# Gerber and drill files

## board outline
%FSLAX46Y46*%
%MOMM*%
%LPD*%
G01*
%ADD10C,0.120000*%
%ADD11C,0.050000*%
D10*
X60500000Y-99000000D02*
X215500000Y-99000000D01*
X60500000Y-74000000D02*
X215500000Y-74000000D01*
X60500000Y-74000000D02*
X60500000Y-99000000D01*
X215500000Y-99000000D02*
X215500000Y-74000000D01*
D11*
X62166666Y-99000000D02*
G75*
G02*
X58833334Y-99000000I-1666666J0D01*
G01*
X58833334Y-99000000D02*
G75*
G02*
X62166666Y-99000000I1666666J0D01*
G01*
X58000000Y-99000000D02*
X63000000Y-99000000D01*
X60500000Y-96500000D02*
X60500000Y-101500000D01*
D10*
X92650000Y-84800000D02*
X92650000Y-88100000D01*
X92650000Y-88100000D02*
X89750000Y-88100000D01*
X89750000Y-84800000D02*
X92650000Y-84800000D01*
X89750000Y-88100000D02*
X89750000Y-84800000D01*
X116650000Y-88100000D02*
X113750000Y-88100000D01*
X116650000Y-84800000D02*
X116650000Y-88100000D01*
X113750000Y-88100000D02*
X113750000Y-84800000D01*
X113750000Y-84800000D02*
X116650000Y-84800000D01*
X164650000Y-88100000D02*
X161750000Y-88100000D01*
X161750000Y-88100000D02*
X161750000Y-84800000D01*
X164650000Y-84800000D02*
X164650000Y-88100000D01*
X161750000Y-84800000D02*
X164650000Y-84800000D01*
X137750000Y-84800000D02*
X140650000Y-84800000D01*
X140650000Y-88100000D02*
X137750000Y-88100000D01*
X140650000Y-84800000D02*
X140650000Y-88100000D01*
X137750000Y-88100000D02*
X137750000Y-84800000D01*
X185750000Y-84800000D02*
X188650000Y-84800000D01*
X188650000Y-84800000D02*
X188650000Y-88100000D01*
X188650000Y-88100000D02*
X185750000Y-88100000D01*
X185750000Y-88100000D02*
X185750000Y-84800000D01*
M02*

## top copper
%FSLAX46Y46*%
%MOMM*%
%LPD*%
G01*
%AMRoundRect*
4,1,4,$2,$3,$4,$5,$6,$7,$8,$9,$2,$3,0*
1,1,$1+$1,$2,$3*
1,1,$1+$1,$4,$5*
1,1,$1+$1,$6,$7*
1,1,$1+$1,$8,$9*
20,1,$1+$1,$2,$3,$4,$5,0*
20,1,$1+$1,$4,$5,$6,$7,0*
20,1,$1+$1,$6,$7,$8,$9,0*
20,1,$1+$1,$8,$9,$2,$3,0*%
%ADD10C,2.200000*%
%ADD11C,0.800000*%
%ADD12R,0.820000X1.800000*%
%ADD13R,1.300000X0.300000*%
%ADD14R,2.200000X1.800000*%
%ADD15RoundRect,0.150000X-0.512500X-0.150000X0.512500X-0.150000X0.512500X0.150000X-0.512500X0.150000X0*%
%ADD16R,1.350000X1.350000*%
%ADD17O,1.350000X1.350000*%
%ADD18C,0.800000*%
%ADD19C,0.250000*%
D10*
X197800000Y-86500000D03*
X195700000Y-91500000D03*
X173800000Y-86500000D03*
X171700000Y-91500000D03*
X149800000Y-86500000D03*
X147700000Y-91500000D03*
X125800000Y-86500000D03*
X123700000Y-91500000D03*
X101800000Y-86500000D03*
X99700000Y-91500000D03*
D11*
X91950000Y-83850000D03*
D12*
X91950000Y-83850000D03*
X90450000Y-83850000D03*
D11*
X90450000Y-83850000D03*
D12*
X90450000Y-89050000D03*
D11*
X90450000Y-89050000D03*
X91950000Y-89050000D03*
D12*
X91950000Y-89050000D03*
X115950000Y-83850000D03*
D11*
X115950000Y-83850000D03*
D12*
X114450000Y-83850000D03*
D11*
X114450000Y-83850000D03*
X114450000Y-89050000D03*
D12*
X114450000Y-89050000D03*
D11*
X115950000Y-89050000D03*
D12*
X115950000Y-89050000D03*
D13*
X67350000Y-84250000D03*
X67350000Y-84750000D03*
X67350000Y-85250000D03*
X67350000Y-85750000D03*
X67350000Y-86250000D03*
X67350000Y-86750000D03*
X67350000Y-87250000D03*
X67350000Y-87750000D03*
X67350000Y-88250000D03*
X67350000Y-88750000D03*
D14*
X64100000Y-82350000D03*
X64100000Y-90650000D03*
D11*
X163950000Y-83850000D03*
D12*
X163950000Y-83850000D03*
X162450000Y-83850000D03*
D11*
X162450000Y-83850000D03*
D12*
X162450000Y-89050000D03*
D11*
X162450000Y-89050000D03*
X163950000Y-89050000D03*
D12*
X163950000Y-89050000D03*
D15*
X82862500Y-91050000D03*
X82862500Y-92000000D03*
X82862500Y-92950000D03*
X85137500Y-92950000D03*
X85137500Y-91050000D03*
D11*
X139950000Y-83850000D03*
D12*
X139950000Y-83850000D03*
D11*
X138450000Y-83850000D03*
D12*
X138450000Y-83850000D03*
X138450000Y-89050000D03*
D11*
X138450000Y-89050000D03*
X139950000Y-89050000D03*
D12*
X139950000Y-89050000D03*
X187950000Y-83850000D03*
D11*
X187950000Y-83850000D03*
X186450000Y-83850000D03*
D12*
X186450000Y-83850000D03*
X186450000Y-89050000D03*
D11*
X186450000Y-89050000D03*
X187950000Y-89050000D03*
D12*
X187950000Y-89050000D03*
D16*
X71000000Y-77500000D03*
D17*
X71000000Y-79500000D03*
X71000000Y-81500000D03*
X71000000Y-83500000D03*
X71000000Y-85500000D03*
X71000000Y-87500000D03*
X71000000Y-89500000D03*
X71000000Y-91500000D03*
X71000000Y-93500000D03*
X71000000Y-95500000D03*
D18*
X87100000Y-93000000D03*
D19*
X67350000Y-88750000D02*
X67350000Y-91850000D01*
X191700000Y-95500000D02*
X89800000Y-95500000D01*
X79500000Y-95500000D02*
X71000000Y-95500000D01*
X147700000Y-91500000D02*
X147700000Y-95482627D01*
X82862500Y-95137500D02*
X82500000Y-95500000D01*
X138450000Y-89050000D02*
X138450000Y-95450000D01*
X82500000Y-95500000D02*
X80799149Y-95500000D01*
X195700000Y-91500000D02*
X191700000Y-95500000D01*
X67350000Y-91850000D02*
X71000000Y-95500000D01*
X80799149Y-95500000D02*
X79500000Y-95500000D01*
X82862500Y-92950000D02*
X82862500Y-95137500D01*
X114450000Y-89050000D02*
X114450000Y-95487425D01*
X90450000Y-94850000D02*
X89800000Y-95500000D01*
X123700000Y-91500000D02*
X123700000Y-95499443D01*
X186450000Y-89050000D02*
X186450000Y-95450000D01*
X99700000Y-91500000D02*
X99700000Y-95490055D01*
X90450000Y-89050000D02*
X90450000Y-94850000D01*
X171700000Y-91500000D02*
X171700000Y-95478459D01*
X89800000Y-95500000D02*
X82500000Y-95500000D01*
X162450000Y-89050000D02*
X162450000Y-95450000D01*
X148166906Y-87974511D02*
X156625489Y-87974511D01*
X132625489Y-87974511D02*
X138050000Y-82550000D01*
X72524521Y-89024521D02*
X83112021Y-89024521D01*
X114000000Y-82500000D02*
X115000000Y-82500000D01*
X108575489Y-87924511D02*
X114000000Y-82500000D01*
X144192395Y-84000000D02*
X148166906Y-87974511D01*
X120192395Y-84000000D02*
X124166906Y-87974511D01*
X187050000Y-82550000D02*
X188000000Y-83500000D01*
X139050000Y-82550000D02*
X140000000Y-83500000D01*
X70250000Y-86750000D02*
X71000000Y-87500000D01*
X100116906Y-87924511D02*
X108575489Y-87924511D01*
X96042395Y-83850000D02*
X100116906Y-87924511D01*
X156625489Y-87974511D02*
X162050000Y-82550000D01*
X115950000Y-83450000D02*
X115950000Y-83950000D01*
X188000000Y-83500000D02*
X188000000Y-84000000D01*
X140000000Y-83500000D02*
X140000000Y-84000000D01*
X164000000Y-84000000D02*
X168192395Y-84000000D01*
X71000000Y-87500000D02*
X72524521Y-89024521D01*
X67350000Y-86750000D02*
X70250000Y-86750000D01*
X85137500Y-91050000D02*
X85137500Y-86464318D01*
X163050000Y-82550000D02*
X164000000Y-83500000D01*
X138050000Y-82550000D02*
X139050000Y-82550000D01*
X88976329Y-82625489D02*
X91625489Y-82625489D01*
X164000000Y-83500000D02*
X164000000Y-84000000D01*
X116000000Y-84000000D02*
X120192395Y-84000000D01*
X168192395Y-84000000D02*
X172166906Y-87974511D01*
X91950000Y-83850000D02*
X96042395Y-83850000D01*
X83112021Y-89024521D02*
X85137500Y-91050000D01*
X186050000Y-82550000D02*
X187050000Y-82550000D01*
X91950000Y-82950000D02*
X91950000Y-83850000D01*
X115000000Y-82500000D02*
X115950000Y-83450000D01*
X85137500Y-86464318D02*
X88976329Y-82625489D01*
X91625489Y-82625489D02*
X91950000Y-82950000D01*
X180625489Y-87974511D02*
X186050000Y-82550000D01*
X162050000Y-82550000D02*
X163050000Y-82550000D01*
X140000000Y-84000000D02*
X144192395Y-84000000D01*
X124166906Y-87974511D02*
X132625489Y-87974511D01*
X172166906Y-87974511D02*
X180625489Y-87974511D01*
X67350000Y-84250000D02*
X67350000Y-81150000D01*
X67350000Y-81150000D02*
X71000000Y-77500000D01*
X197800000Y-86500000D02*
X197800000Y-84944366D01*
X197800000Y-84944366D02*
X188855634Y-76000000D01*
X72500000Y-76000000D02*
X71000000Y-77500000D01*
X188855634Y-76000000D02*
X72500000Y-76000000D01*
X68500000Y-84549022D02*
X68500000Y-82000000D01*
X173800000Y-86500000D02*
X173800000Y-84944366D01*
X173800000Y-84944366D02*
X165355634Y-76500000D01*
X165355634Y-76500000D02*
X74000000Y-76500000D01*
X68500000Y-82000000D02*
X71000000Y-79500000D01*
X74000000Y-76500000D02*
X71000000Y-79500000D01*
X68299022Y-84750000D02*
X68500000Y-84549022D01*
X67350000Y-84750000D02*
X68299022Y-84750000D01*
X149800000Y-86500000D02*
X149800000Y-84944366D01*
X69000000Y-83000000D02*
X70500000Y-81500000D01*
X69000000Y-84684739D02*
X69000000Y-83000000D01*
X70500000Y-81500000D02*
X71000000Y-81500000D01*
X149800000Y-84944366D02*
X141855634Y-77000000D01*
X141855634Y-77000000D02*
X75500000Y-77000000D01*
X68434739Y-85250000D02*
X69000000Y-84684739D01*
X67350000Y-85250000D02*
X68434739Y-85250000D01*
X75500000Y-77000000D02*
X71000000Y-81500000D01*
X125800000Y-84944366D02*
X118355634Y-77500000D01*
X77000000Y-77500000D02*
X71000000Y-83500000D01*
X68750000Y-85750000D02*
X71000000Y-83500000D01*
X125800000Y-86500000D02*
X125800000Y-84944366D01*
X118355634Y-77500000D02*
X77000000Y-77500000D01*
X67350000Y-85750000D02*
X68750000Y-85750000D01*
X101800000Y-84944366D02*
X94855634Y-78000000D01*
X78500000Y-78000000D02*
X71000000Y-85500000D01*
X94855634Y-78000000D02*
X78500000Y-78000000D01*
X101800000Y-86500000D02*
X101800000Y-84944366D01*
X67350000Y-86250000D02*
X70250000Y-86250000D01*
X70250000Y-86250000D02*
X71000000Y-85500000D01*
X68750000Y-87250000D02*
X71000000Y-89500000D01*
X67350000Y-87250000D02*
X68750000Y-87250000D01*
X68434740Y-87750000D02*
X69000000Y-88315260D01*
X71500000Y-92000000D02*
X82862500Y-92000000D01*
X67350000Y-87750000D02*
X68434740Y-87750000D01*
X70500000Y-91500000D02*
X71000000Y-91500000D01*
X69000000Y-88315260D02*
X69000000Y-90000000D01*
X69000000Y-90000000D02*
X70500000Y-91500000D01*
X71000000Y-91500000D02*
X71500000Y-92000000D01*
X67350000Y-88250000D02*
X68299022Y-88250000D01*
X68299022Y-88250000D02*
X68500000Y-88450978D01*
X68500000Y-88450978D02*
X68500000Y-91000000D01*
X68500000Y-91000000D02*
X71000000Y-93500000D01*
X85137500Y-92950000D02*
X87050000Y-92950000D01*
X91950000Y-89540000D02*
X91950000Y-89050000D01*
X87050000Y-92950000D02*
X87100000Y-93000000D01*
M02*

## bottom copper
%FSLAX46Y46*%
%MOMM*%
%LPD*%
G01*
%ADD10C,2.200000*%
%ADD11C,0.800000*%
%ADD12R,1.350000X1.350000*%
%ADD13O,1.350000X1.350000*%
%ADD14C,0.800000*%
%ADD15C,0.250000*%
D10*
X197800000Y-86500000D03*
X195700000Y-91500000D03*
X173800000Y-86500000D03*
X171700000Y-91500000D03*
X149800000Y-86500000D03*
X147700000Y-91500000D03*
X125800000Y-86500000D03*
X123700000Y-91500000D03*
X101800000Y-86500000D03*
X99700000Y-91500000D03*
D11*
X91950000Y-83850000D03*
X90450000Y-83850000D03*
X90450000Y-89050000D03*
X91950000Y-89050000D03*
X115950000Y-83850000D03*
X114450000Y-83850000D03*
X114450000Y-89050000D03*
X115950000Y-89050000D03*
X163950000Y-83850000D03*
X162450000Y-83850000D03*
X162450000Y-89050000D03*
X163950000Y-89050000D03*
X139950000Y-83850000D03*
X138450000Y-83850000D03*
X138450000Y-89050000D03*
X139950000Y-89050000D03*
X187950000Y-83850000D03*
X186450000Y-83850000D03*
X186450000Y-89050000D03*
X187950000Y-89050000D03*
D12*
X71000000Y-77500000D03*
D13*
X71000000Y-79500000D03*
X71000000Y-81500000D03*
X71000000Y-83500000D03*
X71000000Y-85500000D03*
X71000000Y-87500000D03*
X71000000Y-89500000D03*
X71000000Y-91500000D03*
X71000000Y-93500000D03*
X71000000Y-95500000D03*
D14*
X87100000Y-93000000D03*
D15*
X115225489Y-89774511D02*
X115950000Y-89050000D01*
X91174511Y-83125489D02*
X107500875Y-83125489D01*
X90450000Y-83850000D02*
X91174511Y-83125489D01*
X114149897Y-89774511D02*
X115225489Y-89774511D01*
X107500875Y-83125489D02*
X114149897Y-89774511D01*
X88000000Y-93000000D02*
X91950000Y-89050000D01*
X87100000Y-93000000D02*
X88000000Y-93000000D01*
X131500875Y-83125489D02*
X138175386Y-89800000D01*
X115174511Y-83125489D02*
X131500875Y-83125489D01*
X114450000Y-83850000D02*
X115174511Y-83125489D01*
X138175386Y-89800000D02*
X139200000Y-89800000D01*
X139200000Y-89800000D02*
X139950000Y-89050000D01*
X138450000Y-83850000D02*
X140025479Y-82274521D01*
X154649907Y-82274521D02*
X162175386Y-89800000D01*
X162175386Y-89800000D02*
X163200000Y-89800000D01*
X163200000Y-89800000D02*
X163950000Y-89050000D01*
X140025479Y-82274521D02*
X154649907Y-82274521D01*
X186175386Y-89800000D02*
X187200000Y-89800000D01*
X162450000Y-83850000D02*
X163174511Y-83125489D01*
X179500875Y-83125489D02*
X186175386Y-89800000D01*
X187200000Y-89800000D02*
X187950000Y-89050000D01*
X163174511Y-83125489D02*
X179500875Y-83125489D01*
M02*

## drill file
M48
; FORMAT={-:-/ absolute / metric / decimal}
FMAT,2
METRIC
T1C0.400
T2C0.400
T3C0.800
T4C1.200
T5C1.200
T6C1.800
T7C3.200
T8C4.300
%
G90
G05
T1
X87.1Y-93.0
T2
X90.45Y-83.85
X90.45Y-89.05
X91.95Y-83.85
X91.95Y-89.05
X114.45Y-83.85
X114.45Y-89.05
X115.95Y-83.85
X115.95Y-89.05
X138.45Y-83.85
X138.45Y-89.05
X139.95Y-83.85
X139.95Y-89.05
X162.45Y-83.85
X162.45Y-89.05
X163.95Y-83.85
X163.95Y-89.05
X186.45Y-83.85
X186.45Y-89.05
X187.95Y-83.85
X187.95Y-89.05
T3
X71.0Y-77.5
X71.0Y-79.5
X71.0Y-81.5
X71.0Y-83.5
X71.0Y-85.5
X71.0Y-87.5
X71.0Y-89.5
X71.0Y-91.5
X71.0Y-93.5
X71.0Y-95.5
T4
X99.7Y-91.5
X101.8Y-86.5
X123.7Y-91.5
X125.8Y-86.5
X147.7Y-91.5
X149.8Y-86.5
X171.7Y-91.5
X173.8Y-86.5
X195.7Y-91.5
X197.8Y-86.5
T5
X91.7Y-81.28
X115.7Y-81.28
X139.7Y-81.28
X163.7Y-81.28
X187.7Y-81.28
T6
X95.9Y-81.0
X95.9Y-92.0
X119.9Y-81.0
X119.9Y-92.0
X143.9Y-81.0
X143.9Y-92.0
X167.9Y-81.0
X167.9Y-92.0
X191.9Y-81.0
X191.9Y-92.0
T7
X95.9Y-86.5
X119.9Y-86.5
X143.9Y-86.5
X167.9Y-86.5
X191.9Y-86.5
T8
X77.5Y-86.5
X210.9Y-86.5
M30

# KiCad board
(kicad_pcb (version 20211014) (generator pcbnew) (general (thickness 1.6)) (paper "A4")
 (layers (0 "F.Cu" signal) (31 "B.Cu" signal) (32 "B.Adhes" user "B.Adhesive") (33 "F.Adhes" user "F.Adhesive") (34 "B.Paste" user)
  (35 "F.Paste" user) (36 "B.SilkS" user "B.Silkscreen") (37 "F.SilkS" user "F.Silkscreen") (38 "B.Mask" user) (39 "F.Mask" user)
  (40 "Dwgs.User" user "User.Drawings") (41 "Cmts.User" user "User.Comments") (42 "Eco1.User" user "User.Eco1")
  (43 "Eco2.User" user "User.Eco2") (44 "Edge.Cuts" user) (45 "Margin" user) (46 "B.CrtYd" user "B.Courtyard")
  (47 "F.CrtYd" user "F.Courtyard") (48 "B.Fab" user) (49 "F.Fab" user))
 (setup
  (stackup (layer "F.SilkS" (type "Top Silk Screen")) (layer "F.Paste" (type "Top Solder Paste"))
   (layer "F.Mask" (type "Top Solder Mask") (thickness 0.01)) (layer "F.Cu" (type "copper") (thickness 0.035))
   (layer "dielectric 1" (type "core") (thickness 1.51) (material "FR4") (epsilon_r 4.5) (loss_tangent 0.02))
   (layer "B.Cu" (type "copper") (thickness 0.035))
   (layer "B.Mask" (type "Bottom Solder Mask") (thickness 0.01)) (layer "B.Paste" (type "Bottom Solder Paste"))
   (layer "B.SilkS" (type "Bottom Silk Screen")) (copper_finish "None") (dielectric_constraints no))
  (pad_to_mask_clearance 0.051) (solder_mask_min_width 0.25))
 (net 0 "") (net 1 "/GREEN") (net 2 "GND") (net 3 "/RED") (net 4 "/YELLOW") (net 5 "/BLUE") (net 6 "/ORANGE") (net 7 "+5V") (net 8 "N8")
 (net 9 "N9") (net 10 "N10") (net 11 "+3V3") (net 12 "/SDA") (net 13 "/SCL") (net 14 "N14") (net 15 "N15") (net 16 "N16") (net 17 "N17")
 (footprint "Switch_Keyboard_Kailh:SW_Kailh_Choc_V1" (layer "F.Cu") (at 191.9 86.5 -90)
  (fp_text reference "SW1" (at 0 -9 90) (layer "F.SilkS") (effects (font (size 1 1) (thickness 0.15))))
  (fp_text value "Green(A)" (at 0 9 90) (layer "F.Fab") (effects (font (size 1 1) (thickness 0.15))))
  (pad "" np_thru_hole circle locked (at -5.5 0 270) (size 1.8 1.8) (drill 1.8) (layers *.Cu *.Mask))
  (pad "" np_thru_hole circle locked (at 0 0 270) (size 3.2 3.2) (drill 3.2) (layers *.Cu *.Mask))
  (pad "" np_thru_hole circle locked (at -5.22 4.2 270) (size 1.2 1.2) (drill 1.2) (layers *.Cu *.Mask))
  (pad "" np_thru_hole circle locked (at 5.5 0 270) (size 1.8 1.8) (drill 1.8) (layers *.Cu *.Mask))
  (pad "1" thru_hole circle locked (at 0 -5.9 270) (size 2.2 2.2) (drill 1.2) (layers *.Cu "B.Mask") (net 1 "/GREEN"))
  (pad "2" thru_hole circle locked (at 5 -3.8 270) (size 2.2 2.2) (drill 1.2) (layers *.Cu "B.Mask") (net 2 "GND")))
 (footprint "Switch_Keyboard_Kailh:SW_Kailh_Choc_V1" (layer "F.Cu") (at 167.9 86.5 -90)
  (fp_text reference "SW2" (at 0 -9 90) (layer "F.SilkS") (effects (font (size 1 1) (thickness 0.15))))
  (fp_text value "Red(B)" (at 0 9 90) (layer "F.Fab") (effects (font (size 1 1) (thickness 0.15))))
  (pad "" np_thru_hole circle locked (at -5.22 4.2 270) (size 1.2 1.2) (drill 1.2) (layers *.Cu *.Mask))
  (pad "" np_thru_hole circle locked (at 0 0 270) (size 3.2 3.2) (drill 3.2) (layers *.Cu *.Mask))
  (pad "" np_thru_hole circle locked (at -5.5 0 270) (size 1.8 1.8) (drill 1.8) (layers *.Cu *.Mask))
  (pad "" np_thru_hole circle locked (at 5.5 0 270) (size 1.8 1.8) (drill 1.8) (layers *.Cu *.Mask))
  (pad "1" thru_hole circle locked (at 0 -5.9 270) (size 2.2 2.2) (drill 1.2) (layers *.Cu "B.Mask") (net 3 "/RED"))
  (pad "2" thru_hole circle locked (at 5 -3.8 270) (size 2.2 2.2) (drill 1.2) (layers *.Cu "B.Mask") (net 2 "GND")))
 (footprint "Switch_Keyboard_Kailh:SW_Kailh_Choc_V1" (layer "F.Cu") (at 143.9 86.5 -90)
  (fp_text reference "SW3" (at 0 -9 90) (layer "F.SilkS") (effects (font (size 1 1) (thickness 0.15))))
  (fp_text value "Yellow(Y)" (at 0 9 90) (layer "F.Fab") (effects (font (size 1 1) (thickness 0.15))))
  (pad "" np_thru_hole circle locked (at -5.22 4.2 270) (size 1.2 1.2) (drill 1.2) (layers *.Cu *.Mask))
  (pad "" np_thru_hole circle locked (at -5.5 0 270) (size 1.8 1.8) (drill 1.8) (layers *.Cu *.Mask))
  (pad "" np_thru_hole circle locked (at 0 0 270) (size 3.2 3.2) (drill 3.2) (layers *.Cu *.Mask))
  (pad "" np_thru_hole circle locked (at 5.5 0 270) (size 1.8 1.8) (drill 1.8) (layers *.Cu *.Mask))
  (pad "1" thru_hole circle locked (at 0 -5.9 270) (size 2.2 2.2) (drill 1.2) (layers *.Cu "B.Mask") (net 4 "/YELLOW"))
  (pad "2" thru_hole circle locked (at 5 -3.8 270) (size 2.2 2.2) (drill 1.2) (layers *.Cu "B.Mask") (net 2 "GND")))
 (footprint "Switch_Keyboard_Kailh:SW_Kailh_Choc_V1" (layer "F.Cu") (at 119.9 86.5 -90)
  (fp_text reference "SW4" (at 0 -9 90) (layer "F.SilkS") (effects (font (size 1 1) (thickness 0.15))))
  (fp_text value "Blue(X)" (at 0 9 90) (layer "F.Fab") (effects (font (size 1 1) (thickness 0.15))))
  (pad "" np_thru_hole circle locked (at 0 0 270) (size 3.2 3.2) (drill 3.2) (layers *.Cu *.Mask))
  (pad "" np_thru_hole circle locked (at -5.22 4.2 270) (size 1.2 1.2) (drill 1.2) (layers *.Cu *.Mask))
  (pad "" np_thru_hole circle locked (at 5.5 0 270) (size 1.8 1.8) (drill 1.8) (layers *.Cu *.Mask))
  (pad "" np_thru_hole circle locked (at -5.5 0 270) (size 1.8 1.8) (drill 1.8) (layers *.Cu *.Mask))
  (pad "1" thru_hole circle locked (at 0 -5.9 270) (size 2.2 2.2) (drill 1.2) (layers *.Cu "B.Mask") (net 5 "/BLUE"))
  (pad "2" thru_hole circle locked (at 5 -3.8 270) (size 2.2 2.2) (drill 1.2) (layers *.Cu "B.Mask") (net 2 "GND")))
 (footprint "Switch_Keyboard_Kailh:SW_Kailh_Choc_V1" (layer "F.Cu") (at 95.9 86.5 -90)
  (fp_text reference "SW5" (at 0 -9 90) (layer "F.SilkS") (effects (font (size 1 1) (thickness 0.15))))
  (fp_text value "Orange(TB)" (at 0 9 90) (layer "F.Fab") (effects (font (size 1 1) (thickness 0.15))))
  (pad "" np_thru_hole circle locked (at -5.5 0 270) (size 1.8 1.8) (drill 1.8) (layers *.Cu *.Mask))
  (pad "" np_thru_hole circle locked (at 0 0 270) (size 3.2 3.2) (drill 3.2) (layers *.Cu *.Mask))
  (pad "" np_thru_hole circle locked (at -5.22 4.2 270) (size 1.2 1.2) (drill 1.2) (layers *.Cu *.Mask))
  (pad "" np_thru_hole circle locked (at 5.5 0 270) (size 1.8 1.8) (drill 1.8) (layers *.Cu *.Mask))
  (pad "1" thru_hole circle locked (at 0 -5.9 270) (size 2.2 2.2) (drill 1.2) (layers *.Cu "B.Mask") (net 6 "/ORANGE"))
  (pad "2" thru_hole circle locked (at 5 -3.8 270) (size 2.2 2.2) (drill 1.2) (layers *.Cu "B.Mask") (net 2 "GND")))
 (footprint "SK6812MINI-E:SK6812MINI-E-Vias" (layer "F.Cu") (at 91.2 86.5 -90)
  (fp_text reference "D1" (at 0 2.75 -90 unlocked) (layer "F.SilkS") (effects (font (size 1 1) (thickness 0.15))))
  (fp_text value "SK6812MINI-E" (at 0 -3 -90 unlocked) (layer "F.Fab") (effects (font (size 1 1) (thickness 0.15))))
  (fp_line (start -1.7 -1.45) (end 1.6 -1.45) (layer "Edge.Cuts") (width 0.12))
  (fp_line (start 1.6 -1.45) (end 1.6 1.45) (layer "Edge.Cuts") (width 0.12))
  (fp_line (start -1.7 1.45) (end -1.7 -1.45) (layer "Edge.Cuts") (width 0.12))
  (fp_line (start 1.6 1.45) (end -1.7 1.45) (layer "Edge.Cuts") (width 0.12))
  (pad "1" thru_hole circle (at -2.65 -0.75 270) (size 0.8 0.8) (drill 0.4) (layers *.Cu *.Mask) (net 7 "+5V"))
  (pad "1" smd rect (at -2.65 -0.75 270) (size 1.8 0.82) (layers "F.Cu" "F.Paste" "F.Mask") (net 7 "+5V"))
  (pad "2" smd rect (at -2.65 0.75 270) (size 1.8 0.82) (layers "F.Cu" "F.Paste" "F.Mask") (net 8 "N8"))
  (pad "2" thru_hole circle (at -2.65 0.75 270) (size 0.8 0.8) (drill 0.4) (layers *.Cu *.Mask) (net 8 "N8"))
  (pad "3" smd rect (at 2.55 0.75 270) (size 1.8 0.82) (layers "F.Cu" "F.Paste" "F.Mask") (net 2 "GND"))
  (pad "3" thru_hole circle (at 2.55 0.75 270) (size 0.8 0.8) (drill 0.4) (layers *.Cu *.Mask) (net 2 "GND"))
  (pad "4" thru_hole circle (at 2.55 -0.75 270) (size 0.8 0.8) (drill 0.4) (layers *.Cu *.Mask) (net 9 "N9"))
  (pad "4" smd rect (at 2.55 -0.75 270) (size 1.8 0.82) (layers "F.Cu" "F.Paste" "F.Mask") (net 9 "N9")))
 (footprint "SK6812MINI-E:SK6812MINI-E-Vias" (layer "F.Cu") (at 115.2 86.5 -90)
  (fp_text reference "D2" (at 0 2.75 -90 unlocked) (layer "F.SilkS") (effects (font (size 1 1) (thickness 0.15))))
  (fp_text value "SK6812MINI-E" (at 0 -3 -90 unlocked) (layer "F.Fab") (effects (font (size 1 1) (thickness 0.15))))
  (fp_line (start 1.6 -1.45) (end 1.6 1.45) (layer "Edge.Cuts") (width 0.12))
  (fp_line (start -1.7 -1.45) (end 1.6 -1.45) (layer "Edge.Cuts") (width 0.12))
  (fp_line (start 1.6 1.45) (end -1.7 1.45) (layer "Edge.Cuts") (width 0.12))
  (fp_line (start -1.7 1.45) (end -1.7 -1.45) (layer "Edge.Cuts") (width 0.12))
  (pad "1" smd rect (at -2.65 -0.75 270) (size 1.8 0.82) (layers "F.Cu" "F.Paste" "F.Mask") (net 7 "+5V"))
  (pad "1" thru_hole circle (at -2.65 -0.75 270) (size 0.8 0.8) (drill 0.4) (layers *.Cu *.Mask) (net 7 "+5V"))
  (pad "2" smd rect (at -2.65 0.75 270) (size 1.8 0.82) (layers "F.Cu" "F.Paste" "F.Mask") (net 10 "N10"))
  (pad "2" thru_hole circle (at -2.65 0.75 270) (size 0.8 0.8) (drill 0.4) (layers *.Cu *.Mask) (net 10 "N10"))
  (pad "3" thru_hole circle (at 2.55 0.75 270) (size 0.8 0.8) (drill 0.4) (layers *.Cu *.Mask) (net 2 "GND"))
  (pad "3" smd rect (at 2.55 0.75 270) (size 1.8 0.82) (layers "F.Cu" "F.Paste" "F.Mask") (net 2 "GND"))
  (pad "4" thru_hole circle (at 2.55 -0.75 270) (size 0.8 0.8) (drill 0.4) (layers *.Cu *.Mask) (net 8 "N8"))
  (pad "4" smd rect (at 2.55 -0.75 270) (size 1.8 0.82) (layers "F.Cu" "F.Paste" "F.Mask") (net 8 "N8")))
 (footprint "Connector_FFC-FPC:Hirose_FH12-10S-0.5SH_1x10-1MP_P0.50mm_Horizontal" (layer "F.Cu") (at 65.5 86.5 -90)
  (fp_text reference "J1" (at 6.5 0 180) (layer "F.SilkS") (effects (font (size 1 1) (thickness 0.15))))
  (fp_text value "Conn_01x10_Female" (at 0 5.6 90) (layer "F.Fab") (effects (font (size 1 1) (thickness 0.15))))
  (pad "1" smd rect (at -2.25 -1.85 270) (size 0.3 1.3) (layers "F.Cu" "F.Paste" "F.Mask") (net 1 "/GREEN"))
  (pad "2" smd rect (at -1.75 -1.85 270) (size 0.3 1.3) (layers "F.Cu" "F.Paste" "F.Mask") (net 3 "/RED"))
  (pad "3" smd rect (at -1.25 -1.85 270) (size 0.3 1.3) (layers "F.Cu" "F.Paste" "F.Mask") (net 4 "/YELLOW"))
  (pad "4" smd rect (at -0.75 -1.85 270) (size 0.3 1.3) (layers "F.Cu" "F.Paste" "F.Mask") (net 5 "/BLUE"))
  (pad "5" smd rect (at -0.25 -1.85 270) (size 0.3 1.3) (layers "F.Cu" "F.Paste" "F.Mask") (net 6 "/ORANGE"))
  (pad "6" smd rect (at 0.25 -1.85 270) (size 0.3 1.3) (layers "F.Cu" "F.Paste" "F.Mask") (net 7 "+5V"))
  (pad "7" smd rect (at 0.75 -1.85 270) (size 0.3 1.3) (layers "F.Cu" "F.Paste" "F.Mask") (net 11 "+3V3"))
  (pad "8" smd rect (at 1.25 -1.85 270) (size 0.3 1.3) (layers "F.Cu" "F.Paste" "F.Mask") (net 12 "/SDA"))
  (pad "9" smd rect (at 1.75 -1.85 270) (size 0.3 1.3) (layers "F.Cu" "F.Paste" "F.Mask") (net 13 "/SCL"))
  (pad "10" smd rect (at 2.25 -1.85 270) (size 0.3 1.3) (layers "F.Cu" "F.Paste" "F.Mask") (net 2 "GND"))
  (pad "MP" smd rect (at -4.15 1.4 270) (size 1.8 2.2) (layers "F.Cu" "F.Paste" "F.Mask"))
  (pad "MP" smd rect (at 4.15 1.4 270) (size 1.8 2.2) (layers "F.Cu" "F.Paste" "F.Mask")))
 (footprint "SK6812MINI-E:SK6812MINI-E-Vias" (layer "F.Cu") (at 163.2 86.5 -90)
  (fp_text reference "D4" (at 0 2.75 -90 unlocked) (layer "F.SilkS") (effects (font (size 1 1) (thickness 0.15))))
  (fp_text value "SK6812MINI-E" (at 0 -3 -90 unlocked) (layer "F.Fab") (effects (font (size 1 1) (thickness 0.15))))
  (fp_line (start 1.6 -1.45) (end 1.6 1.45) (layer "Edge.Cuts") (width 0.12))
  (fp_line (start 1.6 1.45) (end -1.7 1.45) (layer "Edge.Cuts") (width 0.12))
  (fp_line (start -1.7 -1.45) (end 1.6 -1.45) (layer "Edge.Cuts") (width 0.12))
  (fp_line (start -1.7 1.45) (end -1.7 -1.45) (layer "Edge.Cuts") (width 0.12))
  (pad "1" thru_hole circle (at -2.65 -0.75 270) (size 0.8 0.8) (drill 0.4) (layers *.Cu *.Mask) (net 7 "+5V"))
  (pad "1" smd rect (at -2.65 -0.75 270) (size 1.8 0.82) (layers "F.Cu" "F.Paste" "F.Mask") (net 7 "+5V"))
  (pad "2" smd rect (at -2.65 0.75 270) (size 1.8 0.82) (layers "F.Cu" "F.Paste" "F.Mask") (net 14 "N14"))
  (pad "2" thru_hole circle (at -2.65 0.75 270) (size 0.8 0.8) (drill 0.4) (layers *.Cu *.Mask) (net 14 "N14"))
  (pad "3" smd rect (at 2.55 0.75 270) (size 1.8 0.82) (layers "F.Cu" "F.Paste" "F.Mask") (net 2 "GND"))
  (pad "3" thru_hole circle (at 2.55 0.75 270) (size 0.8 0.8) (drill 0.4) (layers *.Cu *.Mask) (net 2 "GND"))
  (pad "4" thru_hole circle (at 2.55 -0.75 270) (size 0.8 0.8) (drill 0.4) (layers *.Cu *.Mask) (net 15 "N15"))
  (pad "4" smd rect (at 2.55 -0.75 270) (size 1.8 0.82) (layers "F.Cu" "F.Paste" "F.Mask") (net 15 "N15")))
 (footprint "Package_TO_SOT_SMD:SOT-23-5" (layer "F.Cu") (at 84 92)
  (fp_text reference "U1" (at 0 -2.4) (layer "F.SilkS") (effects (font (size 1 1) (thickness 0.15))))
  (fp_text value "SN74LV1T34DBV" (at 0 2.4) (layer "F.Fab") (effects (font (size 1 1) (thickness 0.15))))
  (pad "1" smd roundrect (at -1.1375 -0.95) (size 1.325 0.6) (layers "F.Cu" "F.Paste" "F.Mask") (roundrect_rratio 0.25) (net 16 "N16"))
  (pad "2" smd roundrect (at -1.1375 0) (size 1.325 0.6) (layers "F.Cu" "F.Paste" "F.Mask") (roundrect_rratio 0.25) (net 12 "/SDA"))
  (pad "3" smd roundrect (at -1.1375 0.95) (size 1.325 0.6) (layers "F.Cu" "F.Paste" "F.Mask") (roundrect_rratio 0.25) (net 2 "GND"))
  (pad "4" smd roundrect (at 1.1375 0.95) (size 1.325 0.6) (layers "F.Cu" "F.Paste" "F.Mask") (roundrect_rratio 0.25) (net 9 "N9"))
  (pad "5" smd roundrect (at 1.1375 -0.95) (size 1.325 0.6) (layers "F.Cu" "F.Paste" "F.Mask") (roundrect_rratio 0.25) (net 7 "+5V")))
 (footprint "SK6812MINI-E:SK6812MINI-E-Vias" (layer "F.Cu") (at 139.2 86.5 -90)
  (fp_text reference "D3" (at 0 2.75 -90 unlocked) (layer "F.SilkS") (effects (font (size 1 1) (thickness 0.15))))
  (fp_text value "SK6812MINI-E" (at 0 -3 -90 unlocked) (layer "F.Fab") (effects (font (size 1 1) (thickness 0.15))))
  (fp_line (start -1.7 1.45) (end -1.7 -1.45) (layer "Edge.Cuts") (width 0.12))
  (fp_line (start 1.6 -1.45) (end 1.6 1.45) (layer "Edge.Cuts") (width 0.12))
  (fp_line (start -1.7 -1.45) (end 1.6 -1.45) (layer "Edge.Cuts") (width 0.12))
  (fp_line (start 1.6 1.45) (end -1.7 1.45) (layer "Edge.Cuts") (width 0.12))
  (pad "1" thru_hole circle (at -2.65 -0.75 270) (size 0.8 0.8) (drill 0.4) (layers *.Cu *.Mask) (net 7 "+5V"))
  (pad "1" smd rect (at -2.65 -0.75 270) (size 1.8 0.82) (layers "F.Cu" "F.Paste" "F.Mask") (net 7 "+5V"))
  (pad "2" thru_hole circle (at -2.65 0.75 270) (size 0.8 0.8) (drill 0.4) (layers *.Cu *.Mask) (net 15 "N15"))
  (pad "2" smd rect (at -2.65 0.75 270) (size 1.8 0.82) (layers "F.Cu" "F.Paste" "F.Mask") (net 15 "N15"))
  (pad "3" smd rect (at 2.55 0.75 270) (size 1.8 0.82) (layers "F.Cu" "F.Paste" "F.Mask") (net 2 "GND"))
  (pad "3" thru_hole circle (at 2.55 0.75 270) (size 0.8 0.8) (drill 0.4) (layers *.Cu *.Mask) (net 2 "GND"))
  (pad "4" thru_hole circle (at 2.55 -0.75 270) (size 0.8 0.8) (drill 0.4) (layers *.Cu *.Mask) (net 10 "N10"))
  (pad "4" smd rect (at 2.55 -0.75 270) (size 1.8 0.82) (layers "F.Cu" "F.Paste" "F.Mask") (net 10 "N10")))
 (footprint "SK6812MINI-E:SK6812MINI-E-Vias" (layer "F.Cu") (at 187.2 86.5 -90)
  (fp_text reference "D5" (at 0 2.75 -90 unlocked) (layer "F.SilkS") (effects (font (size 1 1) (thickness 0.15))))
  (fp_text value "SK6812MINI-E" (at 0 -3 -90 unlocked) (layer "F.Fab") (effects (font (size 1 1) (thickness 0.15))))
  (fp_line (start -1.7 1.45) (end -1.7 -1.45) (layer "Edge.Cuts") (width 0.12))
  (fp_line (start -1.7 -1.45) (end 1.6 -1.45) (layer "Edge.Cuts") (width 0.12))
  (fp_line (start 1.6 -1.45) (end 1.6 1.45) (layer "Edge.Cuts") (width 0.12))
  (fp_line (start 1.6 1.45) (end -1.7 1.45) (layer "Edge.Cuts") (width 0.12))
  (pad "1" smd rect (at -2.65 -0.75 270) (size 1.8 0.82) (layers "F.Cu" "F.Paste" "F.Mask") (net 7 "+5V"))
  (pad "1" thru_hole circle (at -2.65 -0.75 270) (size 0.8 0.8) (drill 0.4) (layers *.Cu *.Mask) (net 7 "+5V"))
  (pad "2" thru_hole circle (at -2.65 0.75 270) (size 0.8 0.8) (drill 0.4) (layers *.Cu *.Mask) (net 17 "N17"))
  (pad "2" smd rect (at -2.65 0.75 270) (size 1.8 0.82) (layers "F.Cu" "F.Paste" "F.Mask") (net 17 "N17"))
  (pad "3" smd rect (at 2.55 0.75 270) (size 1.8 0.82) (layers "F.Cu" "F.Paste" "F.Mask") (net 2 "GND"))
  (pad "3" thru_hole circle (at 2.55 0.75 270) (size 0.8 0.8) (drill 0.4) (layers *.Cu *.Mask) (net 2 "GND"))
  (pad "4" thru_hole circle (at 2.55 -0.75 270) (size 0.8 0.8) (drill 0.4) (layers *.Cu *.Mask) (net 14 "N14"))
  (pad "4" smd rect (at 2.55 -0.75 270) (size 1.8 0.82) (layers "F.Cu" "F.Paste" "F.Mask") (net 14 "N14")))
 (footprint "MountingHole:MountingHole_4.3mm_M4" (layer "B.Cu") (at 77.5 86.5 180)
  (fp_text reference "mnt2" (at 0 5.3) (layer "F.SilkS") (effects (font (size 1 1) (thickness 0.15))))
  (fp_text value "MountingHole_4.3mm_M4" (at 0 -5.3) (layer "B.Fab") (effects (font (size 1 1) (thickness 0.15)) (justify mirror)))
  (pad "" np_thru_hole circle (at 0 0 180) (size 4.3 4.3) (drill 4.3) (layers *.Cu *.Mask)))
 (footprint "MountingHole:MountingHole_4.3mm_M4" (layer "B.Cu") (at 210.9 86.5 180)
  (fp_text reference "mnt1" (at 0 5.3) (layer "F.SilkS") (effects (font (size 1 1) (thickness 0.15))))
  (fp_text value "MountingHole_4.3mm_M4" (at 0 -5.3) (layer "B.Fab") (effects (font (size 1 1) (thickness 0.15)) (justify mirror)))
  (pad "" np_thru_hole circle (at 0 0 180) (size 4.3 4.3) (drill 4.3) (layers *.Cu *.Mask)))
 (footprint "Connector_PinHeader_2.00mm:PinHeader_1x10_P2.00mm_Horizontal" (layer "B.Cu") (at 71 77.5 180)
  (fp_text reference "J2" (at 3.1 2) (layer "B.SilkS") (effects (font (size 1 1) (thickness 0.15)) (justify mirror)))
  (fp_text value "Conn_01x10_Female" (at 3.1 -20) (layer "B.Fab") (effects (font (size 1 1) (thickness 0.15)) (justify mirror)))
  (pad "1" thru_hole rect (at 0 0 180) (size 1.35 1.35) (drill 0.8) (layers *.Cu *.Mask) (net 1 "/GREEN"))
  (pad "2" thru_hole oval (at 0 -2 180) (size 1.35 1.35) (drill 0.8) (layers *.Cu *.Mask) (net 3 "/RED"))
  (pad "3" thru_hole oval (at 0 -4 180) (size 1.35 1.35) (drill 0.8) (layers *.Cu *.Mask) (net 4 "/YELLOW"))
  (pad "4" thru_hole oval (at 0 -6 180) (size 1.35 1.35) (drill 0.8) (layers *.Cu *.Mask) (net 5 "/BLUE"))
  (pad "5" thru_hole oval (at 0 -8 180) (size 1.35 1.35) (drill 0.8) (layers *.Cu *.Mask) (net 6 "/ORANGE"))
  (pad "6" thru_hole oval (at 0 -10 180) (size 1.35 1.35) (drill 0.8) (layers *.Cu *.Mask) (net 7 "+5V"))
  (pad "7" thru_hole oval (at 0 -12 180) (size 1.35 1.35) (drill 0.8) (layers *.Cu *.Mask) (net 11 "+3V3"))
  (pad "8" thru_hole oval (at 0 -14 180) (size 1.35 1.35) (drill 0.8) (layers *.Cu *.Mask) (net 12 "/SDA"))
  (pad "9" thru_hole oval (at 0 -16 180) (size 1.35 1.35) (drill 0.8) (layers *.Cu *.Mask) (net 13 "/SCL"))
  (pad "10" thru_hole oval (at 0 -18 180) (size 1.35 1.35) (drill 0.8) (layers *.Cu *.Mask) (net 2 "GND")))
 (gr_line (start 60.5 99) (end 215.5 99) (layer "Edge.Cuts") (width 0.12))
 (gr_line (start 60.5 74) (end 215.5 74) (layer "Edge.Cuts") (width 0.12))
 (gr_line (start 60.5 74) (end 60.5 99) (layer "Edge.Cuts") (width 0.12))
 (gr_line (start 215.5 99) (end 215.5 74) (layer "Edge.Cuts") (width 0.12))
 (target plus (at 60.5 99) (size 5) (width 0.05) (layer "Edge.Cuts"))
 (segment (start 67.35 88.75) (end 67.35 91.85) (width 0.25) (layer "F.Cu") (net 2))
 (segment (start 191.7 95.5) (end 89.8 95.5) (width 0.25) (layer "F.Cu") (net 2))
 (segment (start 79.5 95.5) (end 71 95.5) (width 0.25) (layer "F.Cu") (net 2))
 (segment (start 147.7 91.5) (end 147.7 95.482627) (width 0.25) (layer "F.Cu") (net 2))
 (segment (start 82.8625 95.1375) (end 82.5 95.5) (width 0.25) (layer "F.Cu") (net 2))
 (segment (start 138.45 89.05) (end 138.45 95.45) (width 0.25) (layer "F.Cu") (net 2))
 (segment (start 82.5 95.5) (end 80.799149 95.5) (width 0.25) (layer "F.Cu") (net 2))
 (segment (start 195.7 91.5) (end 191.7 95.5) (width 0.25) (layer "F.Cu") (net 2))
 (segment (start 67.35 91.85) (end 71 95.5) (width 0.25) (layer "F.Cu") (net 2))
 (segment (start 80.799149 95.5) (end 79.5 95.5) (width 0.25) (layer "F.Cu") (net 2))
 (segment (start 82.8625 92.95) (end 82.8625 95.1375) (width 0.25) (layer "F.Cu") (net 2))
 (segment (start 114.45 89.05) (end 114.45 95.487425) (width 0.25) (layer "F.Cu") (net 2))
 (segment (start 90.45 94.85) (end 89.8 95.5) (width 0.25) (layer "F.Cu") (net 2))
 (segment (start 123.7 91.5) (end 123.7 95.499443) (width 0.25) (layer "F.Cu") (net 2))
 (segment (start 186.45 89.05) (end 186.45 95.45) (width 0.25) (layer "F.Cu") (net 2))
 (segment (start 99.7 91.5) (end 99.7 95.490055) (width 0.25) (layer "F.Cu") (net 2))
 (segment (start 90.45 89.05) (end 90.45 94.85) (width 0.25) (layer "F.Cu") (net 2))
 (segment (start 171.7 91.5) (end 171.7 95.478459) (width 0.25) (layer "F.Cu") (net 2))
 (segment (start 89.8 95.5) (end 82.5 95.5) (width 0.25) (layer "F.Cu") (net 2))
 (segment (start 162.45 89.05) (end 162.45 95.45) (width 0.25) (layer "F.Cu") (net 2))
 (segment (start 148.166906 87.974511) (end 156.625489 87.974511) (width 0.25) (layer "F.Cu") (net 7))
 (segment (start 132.625489 87.974511) (end 138.05 82.55) (width 0.25) (layer "F.Cu") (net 7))
 (segment (start 72.524521 89.024521) (end 83.112021 89.024521) (width 0.25) (layer "F.Cu") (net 7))
 (segment (start 114 82.5) (end 115 82.5) (width 0.25) (layer "F.Cu") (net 7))
 (segment (start 108.575489 87.924511) (end 114 82.5) (width 0.25) (layer "F.Cu") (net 7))
 (segment (start 144.192395 84) (end 148.166906 87.974511) (width 0.25) (layer "F.Cu") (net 7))
 (segment (start 120.192395 84) (end 124.166906 87.974511) (width 0.25) (layer "F.Cu") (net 7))
 (segment (start 187.05 82.55) (end 188 83.5) (width 0.25) (layer "F.Cu") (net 7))
 (segment (start 139.05 82.55) (end 140 83.5) (width 0.25) (layer "F.Cu") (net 7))
 (segment (start 70.25 86.75) (end 71 87.5) (width 0.25) (layer "F.Cu") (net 7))
 (segment (start 100.116906 87.924511) (end 108.575489 87.924511) (width 0.25) (layer "F.Cu") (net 7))
 (segment (start 96.042395 83.85) (end 100.116906 87.924511) (width 0.25) (layer "F.Cu") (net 7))
 (segment (start 156.625489 87.974511) (end 162.05 82.55) (width 0.25) (layer "F.Cu") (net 7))
 (segment (start 115.95 83.45) (end 115.95 83.95) (width 0.25) (layer "F.Cu") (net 7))
 (segment (start 188 83.5) (end 188 84) (width 0.25) (layer "F.Cu") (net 7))
 (segment (start 140 83.5) (end 140 84) (width 0.25) (layer "F.Cu") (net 7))
 (segment (start 164 84) (end 168.192395 84) (width 0.25) (layer "F.Cu") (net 7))
 (segment (start 71 87.5) (end 72.524521 89.024521) (width 0.25) (layer "F.Cu") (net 7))
 (segment (start 67.35 86.75) (end 70.25 86.75) (width 0.25) (layer "F.Cu") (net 7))
 (segment (start 85.1375 91.05) (end 85.1375 86.464318) (width 0.25) (layer "F.Cu") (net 7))
 (segment (start 163.05 82.55) (end 164 83.5) (width 0.25) (layer "F.Cu") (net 7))
 (segment (start 138.05 82.55) (end 139.05 82.55) (width 0.25) (layer "F.Cu") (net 7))
 (segment (start 88.976329 82.625489) (end 91.625489 82.625489) (width 0.25) (layer "F.Cu") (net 7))
 (segment (start 164 83.5) (end 164 84) (width 0.25) (layer "F.Cu") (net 7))
 (segment (start 116 84) (end 120.192395 84) (width 0.25) (layer "F.Cu") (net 7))
 (segment (start 168.192395 84) (end 172.166906 87.974511) (width 0.25) (layer "F.Cu") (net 7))
 (segment (start 91.95 83.85) (end 96.042395 83.85) (width 0.25) (layer "F.Cu") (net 7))
 (segment (start 83.112021 89.024521) (end 85.1375 91.05) (width 0.25) (layer "F.Cu") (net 7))
 (segment (start 186.05 82.55) (end 187.05 82.55) (width 0.25) (layer "F.Cu") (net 7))
 (segment (start 91.95 82.95) (end 91.95 83.85) (width 0.25) (layer "F.Cu") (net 7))
 (segment (start 115 82.5) (end 115.95 83.45) (width 0.25) (layer "F.Cu") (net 7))
 (segment (start 85.1375 86.464318) (end 88.976329 82.625489) (width 0.25) (layer "F.Cu") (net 7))
 (segment (start 91.625489 82.625489) (end 91.95 82.95) (width 0.25) (layer "F.Cu") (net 7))
 (segment (start 180.625489 87.974511) (end 186.05 82.55) (width 0.25) (layer "F.Cu") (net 7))
 (segment (start 162.05 82.55) (end 163.05 82.55) (width 0.25) (layer "F.Cu") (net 7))
 (segment (start 140 84) (end 144.192395 84) (width 0.25) (layer "F.Cu") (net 7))
 (segment (start 124.166906 87.974511) (end 132.625489 87.974511) (width 0.25) (layer "F.Cu") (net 7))
 (segment (start 172.166906 87.974511) (end 180.625489 87.974511) (width 0.25) (layer "F.Cu") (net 7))
 (segment (start 67.35 84.25) (end 67.35 81.15) (width 0.25) (layer "F.Cu") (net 1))
 (segment (start 67.35 81.15) (end 71 77.5) (width 0.25) (layer "F.Cu") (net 1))
 (segment (start 197.8 86.5) (end 197.8 84.944366) (width 0.25) (layer "F.Cu") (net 1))
 (segment (start 197.8 84.944366) (end 188.855634 76) (width 0.25) (layer "F.Cu") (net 1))
 (segment (start 72.5 76) (end 71 77.5) (width 0.25) (layer "F.Cu") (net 1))
 (segment (start 188.855634 76) (end 72.5 76) (width 0.25) (layer "F.Cu") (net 1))
 (segment (start 68.5 84.549022) (end 68.5 82) (width 0.25) (layer "F.Cu") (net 3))
 (segment (start 173.8 86.5) (end 173.8 84.944366) (width 0.25) (layer "F.Cu") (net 3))
 (segment (start 173.8 84.944366) (end 165.355634 76.5) (width 0.25) (layer "F.Cu") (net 3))
 (segment (start 165.355634 76.5) (end 74 76.5) (width 0.25) (layer "F.Cu") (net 3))
 (segment (start 68.5 82) (end 71 79.5) (width 0.25) (layer "F.Cu") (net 3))
 (segment (start 74 76.5) (end 71 79.5) (width 0.25) (layer "F.Cu") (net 3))
 (segment (start 68.299022 84.75) (end 68.5 84.549022) (width 0.25) (layer "F.Cu") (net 3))
 (segment (start 67.35 84.75) (end 68.299022 84.75) (width 0.25) (layer "F.Cu") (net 3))
 (segment (start 149.8 86.5) (end 149.8 84.944366) (width 0.25) (layer "F.Cu") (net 4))
 (segment (start 69 83) (end 70.5 81.5) (width 0.25) (layer "F.Cu") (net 4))
 (segment (start 69 84.684739) (end 69 83) (width 0.25) (layer "F.Cu") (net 4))
 (segment (start 70.5 81.5) (end 71 81.5) (width 0.25) (layer "F.Cu") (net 4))
 (segment (start 149.8 84.944366) (end 141.855634 77) (width 0.25) (layer "F.Cu") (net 4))
 (segment (start 141.855634 77) (end 75.5 77) (width 0.25) (layer "F.Cu") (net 4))
 (segment (start 68.434739 85.25) (end 69 84.684739) (width 0.25) (layer "F.Cu") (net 4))
 (segment (start 67.35 85.25) (end 68.434739 85.25) (width 0.25) (layer "F.Cu") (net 4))
 (segment (start 75.5 77) (end 71 81.5) (width 0.25) (layer "F.Cu") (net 4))
 (segment (start 125.8 84.944366) (end 118.355634 77.5) (width 0.25) (layer "F.Cu") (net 5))
 (segment (start 77 77.5) (end 71 83.5) (width 0.25) (layer "F.Cu") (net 5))
 (segment (start 68.75 85.75) (end 71 83.5) (width 0.25) (layer "F.Cu") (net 5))
 (segment (start 125.8 86.5) (end 125.8 84.944366) (width 0.25) (layer "F.Cu") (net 5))
 (segment (start 118.355634 77.5) (end 77 77.5) (width 0.25) (layer "F.Cu") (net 5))
 (segment (start 67.35 85.75) (end 68.75 85.75) (width 0.25) (layer "F.Cu") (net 5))
 (segment (start 101.8 84.944366) (end 94.855634 78) (width 0.25) (layer "F.Cu") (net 6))
 (segment (start 78.5 78) (end 71 85.5) (width 0.25) (layer "F.Cu") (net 6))
 (segment (start 94.855634 78) (end 78.5 78) (width 0.25) (layer "F.Cu") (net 6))
 (segment (start 101.8 86.5) (end 101.8 84.944366) (width 0.25) (layer "F.Cu") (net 6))
 (segment (start 67.35 86.25) (end 70.25 86.25) (width 0.25) (layer "F.Cu") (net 6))
 (segment (start 70.25 86.25) (end 71 85.5) (width 0.25) (layer "F.Cu") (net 6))
 (segment (start 68.75 87.25) (end 71 89.5) (width 0.25) (layer "F.Cu") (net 11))
 (segment (start 67.35 87.25) (end 68.75 87.25) (width 0.25) (layer "F.Cu") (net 11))
 (segment (start 68.43474 87.75) (end 69 88.31526) (width 0.25) (layer "F.Cu") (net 12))
 (segment (start 71.5 92) (end 82.8625 92) (width 0.25) (layer "F.Cu") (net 12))
 (segment (start 67.35 87.75) (end 68.43474 87.75) (width 0.25) (layer "F.Cu") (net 12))
 (segment (start 70.5 91.5) (end 71 91.5) (width 0.25) (layer "F.Cu") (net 12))
 (segment (start 69 88.31526) (end 69 90) (width 0.25) (layer "F.Cu") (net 12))
 (segment (start 69 90) (end 70.5 91.5) (width 0.25) (layer "F.Cu") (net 12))
 (segment (start 71 91.5) (end 71.5 92) (width 0.25) (layer "F.Cu") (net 12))
 (segment (start 67.35 88.25) (end 68.299022 88.25) (width 0.25) (layer "F.Cu") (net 13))
 (segment (start 68.299022 88.25) (end 68.5 88.450978) (width 0.25) (layer "F.Cu") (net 13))
 (segment (start 68.5 88.450978) (end 68.5 91) (width 0.25) (layer "F.Cu") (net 13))
 (segment (start 68.5 91) (end 71 93.5) (width 0.25) (layer "F.Cu") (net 13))
 (segment (start 115.225489 89.774511) (end 115.95 89.05) (width 0.25) (layer "B.Cu") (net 8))
 (segment (start 91.174511 83.125489) (end 107.500875 83.125489) (width 0.25) (layer "B.Cu") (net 8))
 (segment (start 90.45 83.85) (end 91.174511 83.125489) (width 0.25) (layer "B.Cu") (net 8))
 (segment (start 114.149897 89.774511) (end 115.225489 89.774511) (width 0.25) (layer "B.Cu") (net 8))
 (segment (start 107.500875 83.125489) (end 114.149897 89.774511) (width 0.25) (layer "B.Cu") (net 8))
 (segment (start 85.1375 92.95) (end 87.05 92.95) (width 0.25) (layer "F.Cu") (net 9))
 (segment (start 91.95 89.54) (end 91.95 89.05) (width 0.25) (layer "F.Cu") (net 9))
 (segment (start 87.05 92.95) (end 87.1 93) (width 0.25) (layer "F.Cu") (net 9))
 (via (at 87.1 93) (size 0.8) (drill 0.4) (layers "F.Cu" "B.Cu") (free) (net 9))
 (segment (start 88 93) (end 91.95 89.05) (width 0.25) (layer "B.Cu") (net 9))
 (segment (start 87.1 93) (end 88 93) (width 0.25) (layer "B.Cu") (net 9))
 (segment (start 131.500875 83.125489) (end 138.175386 89.8) (width 0.25) (layer "B.Cu") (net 10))
 (segment (start 115.174511 83.125489) (end 131.500875 83.125489) (width 0.25) (layer "B.Cu") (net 10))
 (segment (start 114.45 83.85) (end 115.174511 83.125489) (width 0.25) (layer "B.Cu") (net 10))
 (segment (start 138.175386 89.8) (end 139.2 89.8) (width 0.25) (layer "B.Cu") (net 10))
 (segment (start 139.2 89.8) (end 139.95 89.05) (width 0.25) (layer "B.Cu") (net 10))
 (segment (start 138.45 83.85) (end 140.025479 82.274521) (width 0.25) (layer "B.Cu") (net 15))
 (segment (start 154.649907 82.274521) (end 162.175386 89.8) (width 0.25) (layer "B.Cu") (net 15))
 (segment (start 162.175386 89.8) (end 163.2 89.8) (width 0.25) (layer "B.Cu") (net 15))
 (segment (start 163.2 89.8) (end 163.95 89.05) (width 0.25) (layer "B.Cu") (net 15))
 (segment (start 140.025479 82.274521) (end 154.649907 82.274521) (width 0.25) (layer "B.Cu") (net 15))
 (segment (start 186.175386 89.8) (end 187.2 89.8) (width 0.25) (layer "B.Cu") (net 14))
 (segment (start 162.45 83.85) (end 163.174511 83.125489) (width 0.25) (layer "B.Cu") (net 14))
 (segment (start 179.500875 83.125489) (end 186.175386 89.8) (width 0.25) (layer "B.Cu") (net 14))
 (segment (start 187.2 89.8) (end 187.95 89.05) (width 0.25) (layer "B.Cu") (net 14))
 (segment (start 163.174511 83.125489) (end 179.500875 83.125489) (width 0.25) (layer "B.Cu") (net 14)))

